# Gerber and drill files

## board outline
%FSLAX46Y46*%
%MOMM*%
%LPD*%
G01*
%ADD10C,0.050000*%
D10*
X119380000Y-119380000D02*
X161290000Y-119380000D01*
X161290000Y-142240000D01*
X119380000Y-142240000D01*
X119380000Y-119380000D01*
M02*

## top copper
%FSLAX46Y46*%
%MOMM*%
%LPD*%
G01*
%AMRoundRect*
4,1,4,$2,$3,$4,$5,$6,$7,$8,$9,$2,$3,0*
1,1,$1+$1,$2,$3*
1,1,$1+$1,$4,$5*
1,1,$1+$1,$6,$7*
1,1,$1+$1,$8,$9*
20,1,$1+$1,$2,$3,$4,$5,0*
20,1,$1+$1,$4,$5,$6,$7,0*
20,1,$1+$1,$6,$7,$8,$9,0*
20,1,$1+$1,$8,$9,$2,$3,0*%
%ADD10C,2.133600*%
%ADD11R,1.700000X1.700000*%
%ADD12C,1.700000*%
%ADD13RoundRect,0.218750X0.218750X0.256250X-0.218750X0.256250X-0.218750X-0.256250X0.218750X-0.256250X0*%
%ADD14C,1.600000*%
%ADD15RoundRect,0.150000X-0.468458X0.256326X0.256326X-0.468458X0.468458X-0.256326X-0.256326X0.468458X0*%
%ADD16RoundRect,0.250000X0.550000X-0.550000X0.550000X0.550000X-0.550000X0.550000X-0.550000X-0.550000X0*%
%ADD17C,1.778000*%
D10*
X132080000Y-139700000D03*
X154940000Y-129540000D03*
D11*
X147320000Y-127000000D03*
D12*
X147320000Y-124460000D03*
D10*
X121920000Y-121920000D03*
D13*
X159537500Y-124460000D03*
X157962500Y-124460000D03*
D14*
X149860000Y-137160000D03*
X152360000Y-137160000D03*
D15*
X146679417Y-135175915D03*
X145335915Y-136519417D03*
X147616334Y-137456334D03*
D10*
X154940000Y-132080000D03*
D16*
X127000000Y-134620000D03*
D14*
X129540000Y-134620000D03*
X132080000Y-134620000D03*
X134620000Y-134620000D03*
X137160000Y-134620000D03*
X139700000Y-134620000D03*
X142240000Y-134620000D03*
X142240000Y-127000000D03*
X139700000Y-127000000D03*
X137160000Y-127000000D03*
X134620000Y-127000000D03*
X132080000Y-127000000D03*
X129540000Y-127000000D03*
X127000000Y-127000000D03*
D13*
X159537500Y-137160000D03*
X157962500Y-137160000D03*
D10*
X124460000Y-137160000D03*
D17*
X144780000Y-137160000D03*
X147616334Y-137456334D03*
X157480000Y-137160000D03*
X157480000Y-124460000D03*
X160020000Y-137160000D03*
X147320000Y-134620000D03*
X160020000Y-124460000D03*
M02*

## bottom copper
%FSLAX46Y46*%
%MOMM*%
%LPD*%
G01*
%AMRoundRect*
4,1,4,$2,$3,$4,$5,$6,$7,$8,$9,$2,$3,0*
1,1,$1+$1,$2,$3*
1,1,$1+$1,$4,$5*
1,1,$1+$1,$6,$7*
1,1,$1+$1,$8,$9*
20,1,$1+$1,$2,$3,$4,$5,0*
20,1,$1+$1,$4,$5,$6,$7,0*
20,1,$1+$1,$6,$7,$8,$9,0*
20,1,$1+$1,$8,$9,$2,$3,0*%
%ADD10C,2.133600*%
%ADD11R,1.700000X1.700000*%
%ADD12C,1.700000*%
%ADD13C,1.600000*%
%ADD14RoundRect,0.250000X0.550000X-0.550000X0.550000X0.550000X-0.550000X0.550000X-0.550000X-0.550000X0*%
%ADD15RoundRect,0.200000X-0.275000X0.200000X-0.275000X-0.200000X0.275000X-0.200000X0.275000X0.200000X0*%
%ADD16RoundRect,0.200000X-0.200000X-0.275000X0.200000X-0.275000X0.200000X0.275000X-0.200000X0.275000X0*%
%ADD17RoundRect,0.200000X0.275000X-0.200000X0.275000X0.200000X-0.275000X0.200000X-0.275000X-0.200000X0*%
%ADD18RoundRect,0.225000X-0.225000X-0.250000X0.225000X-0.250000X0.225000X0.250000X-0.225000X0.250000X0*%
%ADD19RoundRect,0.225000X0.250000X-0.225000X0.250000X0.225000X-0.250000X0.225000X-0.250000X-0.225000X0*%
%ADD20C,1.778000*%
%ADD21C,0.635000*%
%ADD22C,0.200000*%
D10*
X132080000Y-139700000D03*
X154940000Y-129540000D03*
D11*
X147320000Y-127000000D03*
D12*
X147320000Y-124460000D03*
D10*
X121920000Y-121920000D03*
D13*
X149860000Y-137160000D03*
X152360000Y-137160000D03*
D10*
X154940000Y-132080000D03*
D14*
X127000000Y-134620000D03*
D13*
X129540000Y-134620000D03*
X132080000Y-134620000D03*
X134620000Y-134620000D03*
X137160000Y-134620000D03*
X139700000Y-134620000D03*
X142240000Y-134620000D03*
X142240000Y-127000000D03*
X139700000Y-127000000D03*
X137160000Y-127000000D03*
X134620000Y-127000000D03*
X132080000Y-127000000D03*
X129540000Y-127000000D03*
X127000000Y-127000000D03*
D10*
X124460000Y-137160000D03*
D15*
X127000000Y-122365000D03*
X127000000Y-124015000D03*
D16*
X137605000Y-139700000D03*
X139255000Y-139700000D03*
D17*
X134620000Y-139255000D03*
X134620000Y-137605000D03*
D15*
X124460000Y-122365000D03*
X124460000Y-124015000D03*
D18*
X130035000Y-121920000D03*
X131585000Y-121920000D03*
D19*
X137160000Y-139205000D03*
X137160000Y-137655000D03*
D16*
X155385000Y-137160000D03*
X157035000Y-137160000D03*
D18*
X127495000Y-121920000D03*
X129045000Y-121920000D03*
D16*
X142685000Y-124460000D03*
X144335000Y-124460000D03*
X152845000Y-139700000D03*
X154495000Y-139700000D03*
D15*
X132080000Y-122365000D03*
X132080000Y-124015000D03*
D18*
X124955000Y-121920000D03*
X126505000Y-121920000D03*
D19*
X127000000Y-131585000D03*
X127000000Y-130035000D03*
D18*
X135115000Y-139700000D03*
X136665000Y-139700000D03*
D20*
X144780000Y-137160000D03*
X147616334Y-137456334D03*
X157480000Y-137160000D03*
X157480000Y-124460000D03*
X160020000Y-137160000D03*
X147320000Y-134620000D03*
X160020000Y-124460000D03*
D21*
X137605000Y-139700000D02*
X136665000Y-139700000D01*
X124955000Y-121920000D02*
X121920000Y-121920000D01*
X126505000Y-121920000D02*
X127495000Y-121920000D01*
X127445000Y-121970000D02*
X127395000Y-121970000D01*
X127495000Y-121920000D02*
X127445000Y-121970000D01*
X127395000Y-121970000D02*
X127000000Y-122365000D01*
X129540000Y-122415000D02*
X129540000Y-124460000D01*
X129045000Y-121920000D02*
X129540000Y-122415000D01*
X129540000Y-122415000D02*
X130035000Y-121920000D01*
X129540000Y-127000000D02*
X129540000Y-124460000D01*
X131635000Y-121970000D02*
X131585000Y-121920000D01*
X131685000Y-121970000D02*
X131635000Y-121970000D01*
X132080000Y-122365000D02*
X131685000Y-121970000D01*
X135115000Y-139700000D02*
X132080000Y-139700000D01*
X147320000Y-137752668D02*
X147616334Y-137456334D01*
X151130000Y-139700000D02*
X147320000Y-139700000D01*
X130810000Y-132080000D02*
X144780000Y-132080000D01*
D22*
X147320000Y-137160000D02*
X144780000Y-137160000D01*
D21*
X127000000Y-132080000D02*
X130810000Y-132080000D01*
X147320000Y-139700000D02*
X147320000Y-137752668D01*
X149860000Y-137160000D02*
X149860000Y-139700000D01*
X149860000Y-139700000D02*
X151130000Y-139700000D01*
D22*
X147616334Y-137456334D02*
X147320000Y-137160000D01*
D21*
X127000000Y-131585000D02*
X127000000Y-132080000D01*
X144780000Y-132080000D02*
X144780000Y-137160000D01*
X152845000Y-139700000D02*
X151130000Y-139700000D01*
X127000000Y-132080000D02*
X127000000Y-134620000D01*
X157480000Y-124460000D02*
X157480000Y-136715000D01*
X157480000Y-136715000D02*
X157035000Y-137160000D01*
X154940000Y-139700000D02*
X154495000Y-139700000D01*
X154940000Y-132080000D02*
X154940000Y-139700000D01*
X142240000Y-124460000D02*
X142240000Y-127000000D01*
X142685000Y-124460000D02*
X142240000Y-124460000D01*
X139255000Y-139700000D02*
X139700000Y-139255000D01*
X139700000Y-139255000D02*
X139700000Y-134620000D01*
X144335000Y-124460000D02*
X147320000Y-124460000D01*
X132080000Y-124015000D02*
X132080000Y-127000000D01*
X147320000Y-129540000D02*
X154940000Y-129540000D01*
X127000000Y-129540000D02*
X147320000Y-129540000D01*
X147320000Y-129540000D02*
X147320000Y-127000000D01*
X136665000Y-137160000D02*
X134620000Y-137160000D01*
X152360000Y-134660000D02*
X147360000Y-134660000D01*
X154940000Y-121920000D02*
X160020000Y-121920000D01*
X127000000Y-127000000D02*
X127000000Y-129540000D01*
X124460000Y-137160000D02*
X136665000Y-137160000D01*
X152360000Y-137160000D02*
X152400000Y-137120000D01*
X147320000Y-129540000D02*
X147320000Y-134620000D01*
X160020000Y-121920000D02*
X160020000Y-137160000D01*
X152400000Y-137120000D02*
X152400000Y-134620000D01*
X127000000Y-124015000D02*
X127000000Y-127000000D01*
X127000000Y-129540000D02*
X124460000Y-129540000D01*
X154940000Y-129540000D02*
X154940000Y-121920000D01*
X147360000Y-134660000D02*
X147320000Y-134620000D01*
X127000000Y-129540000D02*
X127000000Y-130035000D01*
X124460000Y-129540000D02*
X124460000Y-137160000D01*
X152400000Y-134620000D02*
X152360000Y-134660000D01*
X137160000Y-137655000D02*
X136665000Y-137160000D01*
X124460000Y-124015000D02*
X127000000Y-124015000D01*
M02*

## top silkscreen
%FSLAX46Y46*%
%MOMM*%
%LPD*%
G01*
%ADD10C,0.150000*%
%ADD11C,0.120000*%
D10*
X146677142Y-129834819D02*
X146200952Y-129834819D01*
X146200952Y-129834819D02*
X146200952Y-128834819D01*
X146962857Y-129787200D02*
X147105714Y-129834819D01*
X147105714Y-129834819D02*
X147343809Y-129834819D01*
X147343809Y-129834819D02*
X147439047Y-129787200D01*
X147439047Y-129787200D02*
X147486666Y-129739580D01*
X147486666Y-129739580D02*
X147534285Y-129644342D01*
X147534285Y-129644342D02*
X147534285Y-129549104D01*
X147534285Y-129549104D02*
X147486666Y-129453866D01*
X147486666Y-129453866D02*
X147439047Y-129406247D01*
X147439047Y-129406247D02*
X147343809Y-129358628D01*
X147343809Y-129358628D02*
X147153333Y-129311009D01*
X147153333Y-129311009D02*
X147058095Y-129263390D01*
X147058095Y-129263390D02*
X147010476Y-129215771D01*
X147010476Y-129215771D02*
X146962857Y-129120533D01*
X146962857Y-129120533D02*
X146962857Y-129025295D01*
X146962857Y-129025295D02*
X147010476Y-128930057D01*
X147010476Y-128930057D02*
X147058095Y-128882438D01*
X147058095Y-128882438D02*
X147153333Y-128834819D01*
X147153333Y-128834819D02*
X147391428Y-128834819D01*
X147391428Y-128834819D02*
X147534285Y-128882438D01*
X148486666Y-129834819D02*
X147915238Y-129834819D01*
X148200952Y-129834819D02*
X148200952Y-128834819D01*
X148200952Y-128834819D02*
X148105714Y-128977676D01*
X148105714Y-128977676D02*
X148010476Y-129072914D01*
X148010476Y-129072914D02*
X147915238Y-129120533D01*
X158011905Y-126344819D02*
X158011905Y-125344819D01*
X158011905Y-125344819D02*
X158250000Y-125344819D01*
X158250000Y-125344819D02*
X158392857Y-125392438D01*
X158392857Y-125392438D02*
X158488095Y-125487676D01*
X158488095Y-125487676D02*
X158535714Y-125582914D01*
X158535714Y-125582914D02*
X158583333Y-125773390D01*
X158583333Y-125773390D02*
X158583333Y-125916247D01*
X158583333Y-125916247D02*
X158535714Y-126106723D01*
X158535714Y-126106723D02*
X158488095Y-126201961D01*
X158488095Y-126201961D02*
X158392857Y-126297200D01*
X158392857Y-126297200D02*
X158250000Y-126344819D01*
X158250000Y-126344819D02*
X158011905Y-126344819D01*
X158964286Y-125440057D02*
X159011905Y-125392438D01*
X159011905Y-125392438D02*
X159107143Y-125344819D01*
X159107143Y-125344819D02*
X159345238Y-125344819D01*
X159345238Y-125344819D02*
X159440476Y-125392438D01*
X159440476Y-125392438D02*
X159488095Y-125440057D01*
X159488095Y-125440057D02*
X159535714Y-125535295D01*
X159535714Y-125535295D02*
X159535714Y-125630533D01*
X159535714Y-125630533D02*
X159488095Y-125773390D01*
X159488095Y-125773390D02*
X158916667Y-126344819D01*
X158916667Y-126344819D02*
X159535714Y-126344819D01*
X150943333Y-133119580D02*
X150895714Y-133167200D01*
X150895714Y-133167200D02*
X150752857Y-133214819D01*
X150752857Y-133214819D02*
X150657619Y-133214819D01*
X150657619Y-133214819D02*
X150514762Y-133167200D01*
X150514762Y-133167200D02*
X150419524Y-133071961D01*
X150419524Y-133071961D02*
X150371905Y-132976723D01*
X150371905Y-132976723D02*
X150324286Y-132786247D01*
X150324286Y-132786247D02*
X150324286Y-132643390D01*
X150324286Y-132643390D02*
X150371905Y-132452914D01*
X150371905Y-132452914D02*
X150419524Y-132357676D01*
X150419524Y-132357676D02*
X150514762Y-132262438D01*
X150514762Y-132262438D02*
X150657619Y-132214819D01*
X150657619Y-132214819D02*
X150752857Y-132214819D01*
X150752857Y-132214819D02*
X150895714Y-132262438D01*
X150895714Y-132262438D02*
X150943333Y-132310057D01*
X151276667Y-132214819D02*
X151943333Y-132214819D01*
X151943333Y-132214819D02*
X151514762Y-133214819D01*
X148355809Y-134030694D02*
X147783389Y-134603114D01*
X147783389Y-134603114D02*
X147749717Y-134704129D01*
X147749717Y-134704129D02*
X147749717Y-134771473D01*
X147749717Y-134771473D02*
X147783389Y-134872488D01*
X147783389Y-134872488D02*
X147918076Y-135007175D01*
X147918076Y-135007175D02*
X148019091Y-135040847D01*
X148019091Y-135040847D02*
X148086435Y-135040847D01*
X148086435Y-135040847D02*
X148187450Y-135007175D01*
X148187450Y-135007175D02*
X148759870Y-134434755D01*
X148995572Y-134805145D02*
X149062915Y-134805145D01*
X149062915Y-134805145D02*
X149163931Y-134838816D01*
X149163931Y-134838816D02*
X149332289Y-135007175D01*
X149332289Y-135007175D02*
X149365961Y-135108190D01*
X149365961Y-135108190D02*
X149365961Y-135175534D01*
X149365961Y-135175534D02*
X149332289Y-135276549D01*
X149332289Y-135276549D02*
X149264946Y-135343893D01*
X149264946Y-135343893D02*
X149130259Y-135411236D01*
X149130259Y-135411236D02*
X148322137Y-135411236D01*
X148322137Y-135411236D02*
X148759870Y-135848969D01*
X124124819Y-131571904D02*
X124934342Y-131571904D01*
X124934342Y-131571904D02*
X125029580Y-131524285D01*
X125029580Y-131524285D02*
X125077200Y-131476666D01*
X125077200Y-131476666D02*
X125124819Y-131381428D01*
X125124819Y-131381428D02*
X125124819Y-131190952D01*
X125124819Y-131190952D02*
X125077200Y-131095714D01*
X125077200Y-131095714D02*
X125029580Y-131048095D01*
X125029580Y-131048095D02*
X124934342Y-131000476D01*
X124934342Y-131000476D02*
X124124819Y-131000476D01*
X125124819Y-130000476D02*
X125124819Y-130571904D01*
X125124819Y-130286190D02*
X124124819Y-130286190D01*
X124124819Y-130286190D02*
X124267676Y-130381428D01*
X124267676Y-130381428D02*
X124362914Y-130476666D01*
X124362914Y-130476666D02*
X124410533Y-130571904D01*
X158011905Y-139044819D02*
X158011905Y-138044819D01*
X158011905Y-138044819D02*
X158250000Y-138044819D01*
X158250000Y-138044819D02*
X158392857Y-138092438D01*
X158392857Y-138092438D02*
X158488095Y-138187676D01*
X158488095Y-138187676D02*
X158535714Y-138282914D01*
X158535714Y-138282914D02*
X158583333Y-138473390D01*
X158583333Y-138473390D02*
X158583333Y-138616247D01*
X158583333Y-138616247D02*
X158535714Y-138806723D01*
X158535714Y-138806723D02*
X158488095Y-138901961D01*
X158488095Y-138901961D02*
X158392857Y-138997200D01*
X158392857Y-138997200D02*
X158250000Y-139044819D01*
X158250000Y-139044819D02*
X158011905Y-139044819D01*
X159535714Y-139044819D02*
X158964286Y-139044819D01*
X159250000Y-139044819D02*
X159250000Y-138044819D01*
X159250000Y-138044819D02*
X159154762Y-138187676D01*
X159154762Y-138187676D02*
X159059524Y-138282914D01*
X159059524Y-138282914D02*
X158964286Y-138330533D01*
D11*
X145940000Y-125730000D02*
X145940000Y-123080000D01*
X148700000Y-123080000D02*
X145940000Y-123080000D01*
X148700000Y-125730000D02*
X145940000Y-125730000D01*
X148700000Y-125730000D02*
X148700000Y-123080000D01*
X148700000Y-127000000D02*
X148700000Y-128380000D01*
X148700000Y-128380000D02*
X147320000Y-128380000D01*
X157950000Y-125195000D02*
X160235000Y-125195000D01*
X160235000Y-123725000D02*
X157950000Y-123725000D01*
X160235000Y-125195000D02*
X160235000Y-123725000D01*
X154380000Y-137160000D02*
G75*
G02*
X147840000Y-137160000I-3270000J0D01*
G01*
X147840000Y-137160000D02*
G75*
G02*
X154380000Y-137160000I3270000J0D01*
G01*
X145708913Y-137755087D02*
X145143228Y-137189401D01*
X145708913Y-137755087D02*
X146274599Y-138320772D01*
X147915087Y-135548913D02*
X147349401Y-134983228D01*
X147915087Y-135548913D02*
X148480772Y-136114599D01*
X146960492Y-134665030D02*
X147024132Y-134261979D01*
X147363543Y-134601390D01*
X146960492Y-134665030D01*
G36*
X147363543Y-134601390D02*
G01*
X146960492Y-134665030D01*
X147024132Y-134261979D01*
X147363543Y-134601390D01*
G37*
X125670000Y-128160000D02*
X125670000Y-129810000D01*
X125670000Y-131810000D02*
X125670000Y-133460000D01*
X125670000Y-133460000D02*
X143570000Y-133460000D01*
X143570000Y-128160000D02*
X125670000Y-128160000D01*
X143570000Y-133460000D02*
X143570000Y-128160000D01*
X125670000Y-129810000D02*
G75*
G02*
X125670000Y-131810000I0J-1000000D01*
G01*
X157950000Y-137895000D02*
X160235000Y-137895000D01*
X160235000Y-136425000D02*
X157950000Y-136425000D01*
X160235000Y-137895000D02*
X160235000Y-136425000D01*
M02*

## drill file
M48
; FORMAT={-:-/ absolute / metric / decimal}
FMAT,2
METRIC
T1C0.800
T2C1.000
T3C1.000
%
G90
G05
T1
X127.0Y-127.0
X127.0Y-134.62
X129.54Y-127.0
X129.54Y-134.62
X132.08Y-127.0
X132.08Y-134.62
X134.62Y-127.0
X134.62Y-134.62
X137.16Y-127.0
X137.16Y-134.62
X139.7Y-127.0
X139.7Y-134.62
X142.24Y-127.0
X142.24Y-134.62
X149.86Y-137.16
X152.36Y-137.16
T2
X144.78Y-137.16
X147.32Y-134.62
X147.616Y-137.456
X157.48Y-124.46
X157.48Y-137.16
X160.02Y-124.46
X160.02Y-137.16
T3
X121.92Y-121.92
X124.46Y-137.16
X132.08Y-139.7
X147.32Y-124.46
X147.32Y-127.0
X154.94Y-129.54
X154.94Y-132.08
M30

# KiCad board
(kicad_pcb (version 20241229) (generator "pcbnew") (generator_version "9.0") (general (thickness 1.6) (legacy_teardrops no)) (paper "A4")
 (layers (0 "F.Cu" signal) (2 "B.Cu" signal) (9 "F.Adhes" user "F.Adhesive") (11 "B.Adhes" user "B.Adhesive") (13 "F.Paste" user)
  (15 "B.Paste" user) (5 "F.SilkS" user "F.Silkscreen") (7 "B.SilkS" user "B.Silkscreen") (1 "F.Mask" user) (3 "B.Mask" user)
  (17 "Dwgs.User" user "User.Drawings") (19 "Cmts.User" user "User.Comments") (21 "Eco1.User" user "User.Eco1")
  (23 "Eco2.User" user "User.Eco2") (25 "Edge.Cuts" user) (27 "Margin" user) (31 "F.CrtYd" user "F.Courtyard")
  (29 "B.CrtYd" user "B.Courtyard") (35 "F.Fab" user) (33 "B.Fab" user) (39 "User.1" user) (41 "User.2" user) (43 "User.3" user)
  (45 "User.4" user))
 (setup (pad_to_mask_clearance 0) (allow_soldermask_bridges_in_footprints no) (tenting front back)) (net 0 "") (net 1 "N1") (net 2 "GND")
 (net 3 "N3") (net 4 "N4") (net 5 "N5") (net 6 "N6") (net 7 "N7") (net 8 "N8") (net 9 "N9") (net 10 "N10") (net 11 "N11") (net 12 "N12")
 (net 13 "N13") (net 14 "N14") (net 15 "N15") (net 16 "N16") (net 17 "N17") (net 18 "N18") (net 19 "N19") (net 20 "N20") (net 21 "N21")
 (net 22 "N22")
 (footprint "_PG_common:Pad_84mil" (layer "F.Cu") (at 132.08 139.7)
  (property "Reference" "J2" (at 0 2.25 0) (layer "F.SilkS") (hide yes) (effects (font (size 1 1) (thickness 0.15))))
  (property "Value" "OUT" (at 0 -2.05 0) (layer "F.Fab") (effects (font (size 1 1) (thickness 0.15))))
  (pad "1" thru_hole circle (at 0 0) (size 2.1336 2.1336) (drill 1) (layers "*.Cu" "*.Mask") (remove_unused_layers no) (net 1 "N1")))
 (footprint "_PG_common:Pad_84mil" (layer "F.Cu") (at 154.94 129.54)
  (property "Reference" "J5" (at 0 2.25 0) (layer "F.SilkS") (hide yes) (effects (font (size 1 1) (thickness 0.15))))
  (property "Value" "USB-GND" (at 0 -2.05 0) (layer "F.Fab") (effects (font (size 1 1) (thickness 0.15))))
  (pad "1" thru_hole circle (at 0 0) (size 2.1336 2.1336) (drill 1) (layers "*.Cu" "*.Mask") (remove_unused_layers no) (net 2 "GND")))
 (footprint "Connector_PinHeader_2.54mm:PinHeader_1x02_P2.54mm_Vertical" (layer "F.Cu") (at 147.32 127 180)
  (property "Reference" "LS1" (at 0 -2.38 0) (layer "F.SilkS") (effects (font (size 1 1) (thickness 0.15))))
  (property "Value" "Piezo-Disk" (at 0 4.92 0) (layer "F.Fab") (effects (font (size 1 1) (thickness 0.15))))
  (fp_line (start 1.38 1.27) (end 1.38 3.92) (stroke (width 0.12) (type solid)) (layer "F.SilkS"))
  (fp_line (start -1.38 3.92) (end 1.38 3.92) (stroke (width 0.12) (type solid)) (layer "F.SilkS"))
  (fp_line (start -1.38 1.27) (end 1.38 1.27) (stroke (width 0.12) (type solid)) (layer "F.SilkS"))
  (fp_line (start -1.38 1.27) (end -1.38 3.92) (stroke (width 0.12) (type solid)) (layer "F.SilkS"))
  (fp_line (start -1.38 0) (end -1.38 -1.38) (stroke (width 0.12) (type solid)) (layer "F.SilkS"))
  (fp_line (start -1.38 -1.38) (end 0 -1.38) (stroke (width 0.12) (type solid)) (layer "F.SilkS"))
  (pad "1" thru_hole rect (at 0 0 180) (size 1.7 1.7) (drill 1) (layers "*.Cu" "*.Mask") (remove_unused_layers no) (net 2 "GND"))
  (pad "2" thru_hole circle (at 0 2.54 180) (size 1.7 1.7) (drill 1) (layers "*.Cu" "*.Mask") (remove_unused_layers no) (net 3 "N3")))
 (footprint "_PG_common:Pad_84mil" (layer "F.Cu") (at 121.92 121.92)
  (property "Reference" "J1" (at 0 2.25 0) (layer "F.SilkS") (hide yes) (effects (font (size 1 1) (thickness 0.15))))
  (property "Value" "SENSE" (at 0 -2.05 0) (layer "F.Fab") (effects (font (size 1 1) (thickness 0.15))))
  (pad "1" thru_hole circle (at 0 0) (size 2.1336 2.1336) (drill 1) (layers "*.Cu" "*.Mask") (remove_unused_layers no) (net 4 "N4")))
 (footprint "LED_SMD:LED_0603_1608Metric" (layer "F.Cu") (at 158.75 124.46 180)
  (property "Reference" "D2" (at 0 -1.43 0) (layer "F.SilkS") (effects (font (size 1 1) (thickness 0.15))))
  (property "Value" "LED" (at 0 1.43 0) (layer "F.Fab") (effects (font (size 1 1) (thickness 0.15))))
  (fp_line (start 0.8 -0.735) (end -1.485 -0.735) (stroke (width 0.12) (type solid)) (layer "F.SilkS"))
  (fp_line (start -1.485 0.735) (end 0.8 0.735) (stroke (width 0.12) (type solid)) (layer "F.SilkS"))
  (fp_line (start -1.485 -0.735) (end -1.485 0.735) (stroke (width 0.12) (type solid)) (layer "F.SilkS"))
  (pad "1" smd roundrect (at -0.7875 0 180) (size 0.875 0.95) (layers "F.Cu" "F.Mask" "F.Paste") (roundrect_rratio 0.25) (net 2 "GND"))
  (pad "2" smd roundrect (at 0.7875 0 180) (size 0.875 0.95) (layers "F.Cu" "F.Mask" "F.Paste") (roundrect_rratio 0.25) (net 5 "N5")))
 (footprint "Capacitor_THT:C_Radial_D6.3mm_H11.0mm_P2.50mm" (layer "F.Cu") (at 149.86 137.16)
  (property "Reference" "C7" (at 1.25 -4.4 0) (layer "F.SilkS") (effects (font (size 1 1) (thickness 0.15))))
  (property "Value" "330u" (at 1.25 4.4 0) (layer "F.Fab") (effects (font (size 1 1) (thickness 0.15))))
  (fp_circle (center 1.25 0) (end 4.52 0) (stroke (width 0.12) (type solid)) (fill no) (layer "F.SilkS"))
  (pad "1" thru_hole circle (at 0 0) (size 1.6 1.6) (drill 0.8) (layers "*.Cu" "*.Mask") (remove_unused_layers no) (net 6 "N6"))
  (pad "2" thru_hole circle (at 2.5 0) (size 1.6 1.6) (drill 0.8) (layers "*.Cu" "*.Mask") (remove_unused_layers no) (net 2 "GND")))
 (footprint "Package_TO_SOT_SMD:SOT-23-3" (layer "F.Cu") (at 146.812 136.652 -45)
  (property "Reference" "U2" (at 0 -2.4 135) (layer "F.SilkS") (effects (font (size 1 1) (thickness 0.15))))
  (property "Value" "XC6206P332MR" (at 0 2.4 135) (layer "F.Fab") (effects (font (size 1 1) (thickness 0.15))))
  (fp_line (start 0 1.560001) (end -0.8 1.56) (stroke (width 0.12) (type solid)) (layer "F.SilkS"))
  (fp_line (start 0 1.560001) (end 0.8 1.56) (stroke (width 0.12) (type solid)) (layer "F.SilkS"))
  (fp_line (start 0 -1.560001) (end -0.8 -1.56) (stroke (width 0.12) (type solid)) (layer "F.SilkS"))
  (fp_line (start 0 -1.560001) (end 0.8 -1.56) (stroke (width 0.12) (type solid)) (layer "F.SilkS"))
  (fp_poly (pts (xy -1.3 -1.51) (xy -1.54 -1.84) (xy -1.06 -1.84)) (stroke (width 0.12) (type solid)) (fill yes) (layer "F.SilkS"))
  (pad "1" smd roundrect (at -1.1375 -0.949999 315) (size 1.325 0.6) (layers "F.Cu" "F.Mask" "F.Paste") (roundrect_rratio 0.25)
   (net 2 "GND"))
  (pad "2" smd roundrect (at -1.1375 0.949999 315) (size 1.325 0.6) (layers "F.Cu" "F.Mask" "F.Paste") (roundrect_rratio 0.25) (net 6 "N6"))
  (pad "3" smd roundrect (at 1.1375 0 315) (size 1.325 0.6) (layers "F.Cu" "F.Mask" "F.Paste") (roundrect_rratio 0.25) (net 6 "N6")))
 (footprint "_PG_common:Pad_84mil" (layer "F.Cu") (at 154.94 132.08)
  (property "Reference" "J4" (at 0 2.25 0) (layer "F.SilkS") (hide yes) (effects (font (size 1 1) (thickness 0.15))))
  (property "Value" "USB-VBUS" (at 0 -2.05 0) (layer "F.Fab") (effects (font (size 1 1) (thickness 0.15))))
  (pad "1" thru_hole circle (at 0 0) (size 2.1336 2.1336) (drill 1) (layers "*.Cu" "*.Mask") (remove_unused_layers no) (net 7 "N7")))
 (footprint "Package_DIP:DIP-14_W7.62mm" (layer "F.Cu") (at 127 134.62 90)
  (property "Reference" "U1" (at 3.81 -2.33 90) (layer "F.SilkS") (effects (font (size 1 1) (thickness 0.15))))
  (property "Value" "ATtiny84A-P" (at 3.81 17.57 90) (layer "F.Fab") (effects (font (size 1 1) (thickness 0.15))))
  (fp_line (start 6.46 -1.33) (end 4.81 -1.33) (stroke (width 0.12) (type solid)) (layer "F.SilkS"))
  (fp_line (start 2.81 -1.33) (end 1.16 -1.33) (stroke (width 0.12) (type solid)) (layer "F.SilkS"))
  (fp_line (start 1.16 -1.33) (end 1.16 16.57) (stroke (width 0.12) (type solid)) (layer "F.SilkS"))
  (fp_line (start 6.46 16.57) (end 6.46 -1.33) (stroke (width 0.12) (type solid)) (layer "F.SilkS"))
  (fp_line (start 1.16 16.57) (end 6.46 16.57) (stroke (width 0.12) (type solid)) (layer "F.SilkS"))
  (fp_arc (start 4.81 -1.33) (mid 3.81 -0.33) (end 2.81 -1.33) (stroke (width 0.12) (type solid)) (layer "F.SilkS"))
  (pad "1" thru_hole roundrect (at 0 0 90) (size 1.6 1.6) (drill 0.8) (layers "*.Cu" "*.Mask") (remove_unused_layers no)
   (roundrect_rratio 0.15625) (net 6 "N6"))
  (pad "2" thru_hole circle (at 0 2.54 90) (size 1.6 1.6) (drill 0.8) (layers "*.Cu" "*.Mask") (remove_unused_layers no) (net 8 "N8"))
  (pad "3" thru_hole circle (at 0 5.08 90) (size 1.6 1.6) (drill 0.8) (layers "*.Cu" "*.Mask") (remove_unused_layers no) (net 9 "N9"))
  (pad "4" thru_hole circle (at 0 7.62 90) (size 1.6 1.6) (drill 0.8) (layers "*.Cu" "*.Mask") (remove_unused_layers no) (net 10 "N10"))
  (pad "5" thru_hole circle (at 0 10.16 90) (size 1.6 1.6) (drill 0.8) (layers "*.Cu" "*.Mask") (remove_unused_layers no) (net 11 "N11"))
  (pad "6" thru_hole circle (at 0 12.7 90) (size 1.6 1.6) (drill 0.8) (layers "*.Cu" "*.Mask") (remove_unused_layers no) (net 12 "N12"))
  (pad "7" thru_hole circle (at 0 15.24 90) (size 1.6 1.6) (drill 0.8) (layers "*.Cu" "*.Mask") (remove_unused_layers no) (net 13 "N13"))
  (pad "8" thru_hole circle (at 7.62 15.24 90) (size 1.6 1.6) (drill 0.8) (layers "*.Cu" "*.Mask") (remove_unused_layers no) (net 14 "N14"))
  (pad "9" thru_hole circle (at 7.62 12.7 90) (size 1.6 1.6) (drill 0.8) (layers "*.Cu" "*.Mask") (remove_unused_layers no) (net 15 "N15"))
  (pad "10" thru_hole circle (at 7.62 10.16 90) (size 1.6 1.6) (drill 0.8) (layers "*.Cu" "*.Mask") (remove_unused_layers no) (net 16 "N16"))
  (pad "11" thru_hole circle (at 7.62 7.62 90) (size 1.6 1.6) (drill 0.8) (layers "*.Cu" "*.Mask") (remove_unused_layers no) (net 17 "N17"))
  (pad "12" thru_hole circle (at 7.62 5.08 90) (size 1.6 1.6) (drill 0.8) (layers "*.Cu" "*.Mask") (remove_unused_layers no) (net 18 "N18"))
  (pad "13" thru_hole circle (at 7.62 2.54 90) (size 1.6 1.6) (drill 0.8) (layers "*.Cu" "*.Mask") (remove_unused_layers no) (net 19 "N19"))
  (pad "14" thru_hole circle (at 7.62 0 90) (size 1.6 1.6) (drill 0.8) (layers "*.Cu" "*.Mask") (remove_unused_layers no) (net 2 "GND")))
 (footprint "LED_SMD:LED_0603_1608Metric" (layer "F.Cu") (at 158.75 137.16 180)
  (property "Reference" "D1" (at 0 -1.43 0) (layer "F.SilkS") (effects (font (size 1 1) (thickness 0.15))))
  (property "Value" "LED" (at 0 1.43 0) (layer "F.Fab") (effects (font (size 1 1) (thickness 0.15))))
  (fp_line (start 0.8 -0.735) (end -1.485 -0.735) (stroke (width 0.12) (type solid)) (layer "F.SilkS"))
  (fp_line (start -1.485 0.735) (end 0.8 0.735) (stroke (width 0.12) (type solid)) (layer "F.SilkS"))
  (fp_line (start -1.485 -0.735) (end -1.485 0.735) (stroke (width 0.12) (type solid)) (layer "F.SilkS"))
  (pad "1" smd roundrect (at -0.7875 0 180) (size 0.875 0.95) (layers "F.Cu" "F.Mask" "F.Paste") (roundrect_rratio 0.25) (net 2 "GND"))
  (pad "2" smd roundrect (at 0.7875 0 180) (size 0.875 0.95) (layers "F.Cu" "F.Mask" "F.Paste") (roundrect_rratio 0.25) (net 5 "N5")))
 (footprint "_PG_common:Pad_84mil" (layer "F.Cu") (at 124.46 137.16)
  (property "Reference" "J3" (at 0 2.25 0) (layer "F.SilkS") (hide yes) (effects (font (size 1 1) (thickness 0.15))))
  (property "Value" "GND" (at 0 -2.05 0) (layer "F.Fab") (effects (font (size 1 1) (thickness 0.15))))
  (pad "1" thru_hole circle (at 0 0) (size 2.1336 2.1336) (drill 1) (layers "*.Cu" "*.Mask") (remove_unused_layers no) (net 2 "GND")))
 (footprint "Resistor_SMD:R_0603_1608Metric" (layer "B.Cu") (at 127 123.19 -90)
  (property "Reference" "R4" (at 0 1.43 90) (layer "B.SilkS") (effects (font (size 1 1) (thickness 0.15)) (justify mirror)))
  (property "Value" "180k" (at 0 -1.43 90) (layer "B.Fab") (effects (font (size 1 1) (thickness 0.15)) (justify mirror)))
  (pad "1" smd roundrect (at -0.825 0 270) (size 0.8 0.95) (layers "B.Cu" "B.Mask" "B.Paste") (roundrect_rratio 0.25) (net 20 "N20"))
  (pad "2" smd roundrect (at 0.825 0 270) (size 0.8 0.95) (layers "B.Cu" "B.Mask" "B.Paste") (roundrect_rratio 0.25) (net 2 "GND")))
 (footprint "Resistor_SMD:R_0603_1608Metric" (layer "B.Cu") (at 138.43 139.7)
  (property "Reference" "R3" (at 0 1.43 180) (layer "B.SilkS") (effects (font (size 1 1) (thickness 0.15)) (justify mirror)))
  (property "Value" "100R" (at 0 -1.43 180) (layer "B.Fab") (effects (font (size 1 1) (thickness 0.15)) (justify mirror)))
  (pad "1" smd roundrect (at -0.825 0) (size 0.8 0.95) (layers "B.Cu" "B.Mask" "B.Paste") (roundrect_rratio 0.25) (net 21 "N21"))
  (pad "2" smd roundrect (at 0.825 0) (size 0.8 0.95) (layers "B.Cu" "B.Mask" "B.Paste") (roundrect_rratio 0.25) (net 12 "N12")))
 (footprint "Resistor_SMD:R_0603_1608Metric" (layer "B.Cu") (at 134.62 138.43 90)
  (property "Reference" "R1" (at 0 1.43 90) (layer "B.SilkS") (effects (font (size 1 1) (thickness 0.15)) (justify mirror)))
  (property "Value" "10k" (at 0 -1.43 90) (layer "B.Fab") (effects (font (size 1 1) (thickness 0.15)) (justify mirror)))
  (pad "1" smd roundrect (at -0.825 0 90) (size 0.8 0.95) (layers "B.Cu" "B.Mask" "B.Paste") (roundrect_rratio 0.25) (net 1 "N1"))
  (pad "2" smd roundrect (at 0.825 0 90) (size 0.8 0.95) (layers "B.Cu" "B.Mask" "B.Paste") (roundrect_rratio 0.25) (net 2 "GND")))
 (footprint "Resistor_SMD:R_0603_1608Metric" (layer "B.Cu") (at 124.46 123.19 -90)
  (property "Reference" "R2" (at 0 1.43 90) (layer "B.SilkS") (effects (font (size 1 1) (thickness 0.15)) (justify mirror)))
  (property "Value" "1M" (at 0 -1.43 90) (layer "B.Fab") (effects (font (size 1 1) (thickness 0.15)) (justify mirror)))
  (pad "1" smd roundrect (at -0.825 0 270) (size 0.8 0.95) (layers "B.Cu" "B.Mask" "B.Paste") (roundrect_rratio 0.25) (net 4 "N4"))
  (pad "2" smd roundrect (at 0.825 0 270) (size 0.8 0.95) (layers "B.Cu" "B.Mask" "B.Paste") (roundrect_rratio 0.25) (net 2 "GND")))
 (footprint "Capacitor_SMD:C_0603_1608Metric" (layer "B.Cu") (at 130.81 121.92)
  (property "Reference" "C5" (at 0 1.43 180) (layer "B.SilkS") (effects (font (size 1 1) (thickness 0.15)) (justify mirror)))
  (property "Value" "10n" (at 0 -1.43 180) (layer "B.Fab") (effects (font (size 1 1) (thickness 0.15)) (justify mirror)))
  (pad "1" smd roundrect (at -0.775 0) (size 0.9 0.95) (layers "B.Cu" "B.Mask" "B.Paste") (roundrect_rratio 0.25) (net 19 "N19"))
  (pad "2" smd roundrect (at 0.775 0) (size 0.9 0.95) (layers "B.Cu" "B.Mask" "B.Paste") (roundrect_rratio 0.25) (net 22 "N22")))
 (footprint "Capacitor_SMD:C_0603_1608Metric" (layer "B.Cu") (at 137.16 138.43 90)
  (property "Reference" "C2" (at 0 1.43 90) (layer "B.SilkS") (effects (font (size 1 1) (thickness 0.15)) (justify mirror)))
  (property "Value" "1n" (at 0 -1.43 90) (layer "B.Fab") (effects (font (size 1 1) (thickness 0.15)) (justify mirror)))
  (pad "1" smd roundrect (at -0.775 0 90) (size 0.9 0.95) (layers "B.Cu" "B.Mask" "B.Paste") (roundrect_rratio 0.25) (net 21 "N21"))
  (pad "2" smd roundrect (at 0.775 0 90) (size 0.9 0.95) (layers "B.Cu" "B.Mask" "B.Paste") (roundrect_rratio 0.25) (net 2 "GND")))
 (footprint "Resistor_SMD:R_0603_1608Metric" (layer "B.Cu") (at 156.21 137.16)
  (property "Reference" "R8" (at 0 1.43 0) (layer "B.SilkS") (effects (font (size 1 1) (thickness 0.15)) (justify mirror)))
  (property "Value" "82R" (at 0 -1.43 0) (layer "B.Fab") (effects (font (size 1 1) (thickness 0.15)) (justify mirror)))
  (pad "1" smd roundrect (at -0.825 0) (size 0.8 0.95) (layers "B.Cu" "B.Mask" "B.Paste") (roundrect_rratio 0.25) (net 7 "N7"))
  (pad "2" smd roundrect (at 0.825 0) (size 0.8 0.95) (layers "B.Cu" "B.Mask" "B.Paste") (roundrect_rratio 0.25) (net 5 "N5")))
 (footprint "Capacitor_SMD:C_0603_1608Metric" (layer "B.Cu") (at 128.27 121.92)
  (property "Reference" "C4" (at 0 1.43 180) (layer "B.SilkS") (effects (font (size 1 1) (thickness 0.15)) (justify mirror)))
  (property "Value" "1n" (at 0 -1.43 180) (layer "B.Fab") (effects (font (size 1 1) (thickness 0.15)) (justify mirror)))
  (pad "1" smd roundrect (at -0.775 0) (size 0.9 0.95) (layers "B.Cu" "B.Mask" "B.Paste") (roundrect_rratio 0.25) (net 20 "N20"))
  (pad "2" smd roundrect (at 0.775 0) (size 0.9 0.95) (layers "B.Cu" "B.Mask" "B.Paste") (roundrect_rratio 0.25) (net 19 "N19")))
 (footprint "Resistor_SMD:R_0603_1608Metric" (layer "B.Cu") (at 143.51 124.46)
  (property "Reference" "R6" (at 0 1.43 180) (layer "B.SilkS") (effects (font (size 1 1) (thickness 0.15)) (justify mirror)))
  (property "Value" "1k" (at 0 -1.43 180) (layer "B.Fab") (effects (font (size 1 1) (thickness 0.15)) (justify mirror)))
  (pad "1" smd roundrect (at -0.825 0) (size 0.8 0.95) (layers "B.Cu" "B.Mask" "B.Paste") (roundrect_rratio 0.25) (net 14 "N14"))
  (pad "2" smd roundrect (at 0.825 0) (size 0.8 0.95) (layers "B.Cu" "B.Mask" "B.Paste") (roundrect_rratio 0.25) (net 3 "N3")))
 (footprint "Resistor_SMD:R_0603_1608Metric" (layer "B.Cu") (at 153.67 139.7)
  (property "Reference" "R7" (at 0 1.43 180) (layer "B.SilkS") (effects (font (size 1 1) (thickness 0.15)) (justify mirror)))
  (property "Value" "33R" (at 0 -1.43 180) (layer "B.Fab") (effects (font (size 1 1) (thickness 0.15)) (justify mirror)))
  (pad "1" smd roundrect (at -0.825 0) (size 0.8 0.95) (layers "B.Cu" "B.Mask" "B.Paste") (roundrect_rratio 0.25) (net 6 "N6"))
  (pad "2" smd roundrect (at 0.825 0) (size 0.8 0.95) (layers "B.Cu" "B.Mask" "B.Paste") (roundrect_rratio 0.25) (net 7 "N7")))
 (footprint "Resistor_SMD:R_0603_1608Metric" (layer "B.Cu") (at 132.08 123.19 -90)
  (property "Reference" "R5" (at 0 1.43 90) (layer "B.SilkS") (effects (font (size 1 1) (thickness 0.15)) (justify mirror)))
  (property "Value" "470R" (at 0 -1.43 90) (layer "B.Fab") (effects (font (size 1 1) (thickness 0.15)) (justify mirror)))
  (pad "1" smd roundrect (at -0.825 0 270) (size 0.8 0.95) (layers "B.Cu" "B.Mask" "B.Paste") (roundrect_rratio 0.25) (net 22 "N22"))
  (pad "2" smd roundrect (at 0.825 0 270) (size 0.8 0.95) (layers "B.Cu" "B.Mask" "B.Paste") (roundrect_rratio 0.25) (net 18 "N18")))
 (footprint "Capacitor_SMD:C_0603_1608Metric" (layer "B.Cu") (at 125.73 121.92)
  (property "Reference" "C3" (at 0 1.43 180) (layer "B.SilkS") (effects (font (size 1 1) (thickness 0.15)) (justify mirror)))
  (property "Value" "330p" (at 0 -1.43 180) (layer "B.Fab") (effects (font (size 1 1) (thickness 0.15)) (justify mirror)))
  (pad "1" smd roundrect (at -0.775 0) (size 0.9 0.95) (layers "B.Cu" "B.Mask" "B.Paste") (roundrect_rratio 0.25) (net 4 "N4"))
  (pad "2" smd roundrect (at 0.775 0) (size 0.9 0.95) (layers "B.Cu" "B.Mask" "B.Paste") (roundrect_rratio 0.25) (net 20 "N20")))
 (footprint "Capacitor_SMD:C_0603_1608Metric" (layer "B.Cu") (at 127 130.81 90)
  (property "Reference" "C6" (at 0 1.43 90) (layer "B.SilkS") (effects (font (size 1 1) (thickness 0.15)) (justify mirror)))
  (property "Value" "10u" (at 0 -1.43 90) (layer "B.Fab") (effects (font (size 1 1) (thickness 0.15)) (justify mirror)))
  (pad "1" smd roundrect (at -0.775 0 90) (size 0.9 0.95) (layers "B.Cu" "B.Mask" "B.Paste") (roundrect_rratio 0.25) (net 6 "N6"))
  (pad "2" smd roundrect (at 0.775 0 90) (size 0.9 0.95) (layers "B.Cu" "B.Mask" "B.Paste") (roundrect_rratio 0.25) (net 2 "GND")))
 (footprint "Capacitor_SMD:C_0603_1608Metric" (layer "B.Cu") (at 135.89 139.7)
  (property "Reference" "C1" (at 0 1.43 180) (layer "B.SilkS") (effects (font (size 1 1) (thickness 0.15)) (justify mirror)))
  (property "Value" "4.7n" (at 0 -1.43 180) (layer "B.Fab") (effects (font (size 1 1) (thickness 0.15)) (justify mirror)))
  (pad "1" smd roundrect (at -0.775 0) (size 0.9 0.95) (layers "B.Cu" "B.Mask" "B.Paste") (roundrect_rratio 0.25) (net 1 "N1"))
  (pad "2" smd roundrect (at 0.775 0) (size 0.9 0.95) (layers "B.Cu" "B.Mask" "B.Paste") (roundrect_rratio 0.25) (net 21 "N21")))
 (gr_rect (start 119.38 119.38) (end 161.29 142.24) (stroke (width 0.05) (type default)) (fill no) (layer "Edge.Cuts"))
 (segment (start 137.605 139.7) (end 136.665 139.7) (width 0.635) (layer "B.Cu") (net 21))
 (segment (start 124.955 121.92) (end 121.92 121.92) (width 0.635) (layer "B.Cu") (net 4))
 (segment (start 126.505 121.92) (end 127.495 121.92) (width 0.635) (layer "B.Cu") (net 20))
 (segment (start 127.445 121.97) (end 127.395 121.97) (width 0.635) (layer "B.Cu") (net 20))
 (segment (start 127.495 121.92) (end 127.445 121.97) (width 0.635) (layer "B.Cu") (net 20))
 (segment (start 127.395 121.97) (end 127 122.365) (width 0.635) (layer "B.Cu") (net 20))
 (segment (start 129.54 122.415) (end 129.54 124.46) (width 0.635) (layer "B.Cu") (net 19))
 (segment (start 129.045 121.92) (end 129.54 122.415) (width 0.635) (layer "B.Cu") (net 19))
 (segment (start 129.54 122.415) (end 130.035 121.92) (width 0.635) (layer "B.Cu") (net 19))
 (segment (start 129.54 127) (end 129.54 124.46) (width 0.635) (layer "B.Cu") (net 19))
 (segment (start 131.635 121.97) (end 131.585 121.92) (width 0.635) (layer "B.Cu") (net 22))
 (segment (start 131.685 121.97) (end 131.635 121.97) (width 0.635) (layer "B.Cu") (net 22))
 (segment (start 132.08 122.365) (end 131.685 121.97) (width 0.635) (layer "B.Cu") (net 22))
 (segment (start 135.115 139.7) (end 132.08 139.7) (width 0.635) (layer "B.Cu") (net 1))
 (via (at 144.78 137.16) (size 1.778) (drill 1) (layers "F.Cu" "B.Cu") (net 6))
 (via (at 147.616334 137.456334) (size 1.778) (drill 1) (layers "F.Cu" "B.Cu") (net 6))
 (segment (start 147.32 137.752668) (end 147.616334 137.456334) (width 0.635) (layer "B.Cu") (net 6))
 (segment (start 151.13 139.7) (end 147.32 139.7) (width 0.635) (layer "B.Cu") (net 6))
 (segment (start 130.81 132.08) (end 144.78 132.08) (width 0.635) (layer "B.Cu") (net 6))
 (segment (start 147.32 137.16) (end 144.78 137.16) (width 0.2) (layer "B.Cu") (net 6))
 (segment (start 127 132.08) (end 130.81 132.08) (width 0.635) (layer "B.Cu") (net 6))
 (segment (start 147.32 139.7) (end 147.32 137.752668) (width 0.635) (layer "B.Cu") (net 6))
 (segment (start 149.86 137.16) (end 149.86 139.7) (width 0.635) (layer "B.Cu") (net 6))
 (segment (start 149.86 139.7) (end 151.13 139.7) (width 0.635) (layer "B.Cu") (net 6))
 (segment (start 147.616334 137.456334) (end 147.32 137.16) (width 0.2) (layer "B.Cu") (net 6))
 (segment (start 127 131.585) (end 127 132.08) (width 0.635) (layer "B.Cu") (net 6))
 (segment (start 144.78 132.08) (end 144.78 137.16) (width 0.635) (layer "B.Cu") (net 6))
 (segment (start 152.845 139.7) (end 151.13 139.7) (width 0.635) (layer "B.Cu") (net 6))
 (segment (start 127 132.08) (end 127 134.62) (width 0.635) (layer "B.Cu") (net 6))
 (via (at 157.48 137.16) (size 1.778) (drill 1) (layers "F.Cu" "B.Cu") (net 5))
 (via (at 157.48 124.46) (size 1.778) (drill 1) (layers "F.Cu" "B.Cu") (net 5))
 (segment (start 157.48 124.46) (end 157.48 136.715) (width 0.635) (layer "B.Cu") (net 5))
 (segment (start 157.48 136.715) (end 157.035 137.16) (width 0.635) (layer "B.Cu") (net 5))
 (segment (start 154.94 139.7) (end 154.495 139.7) (width 0.635) (layer "B.Cu") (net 7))
 (segment (start 154.94 132.08) (end 154.94 139.7) (width 0.635) (layer "B.Cu") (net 7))
 (segment (start 142.24 124.46) (end 142.24 127) (width 0.635) (layer "B.Cu") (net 14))
 (segment (start 142.685 124.46) (end 142.24 124.46) (width 0.635) (layer "B.Cu") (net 14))
 (segment (start 139.255 139.7) (end 139.7 139.255) (width 0.635) (layer "B.Cu") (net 12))
 (segment (start 139.7 139.255) (end 139.7 134.62) (width 0.635) (layer "B.Cu") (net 12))
 (segment (start 144.335 124.46) (end 147.32 124.46) (width 0.635) (layer "B.Cu") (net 3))
 (segment (start 132.08 124.015) (end 132.08 127) (width 0.635) (layer "B.Cu") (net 18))
 (via (at 160.02 137.16) (size 1.778) (drill 1) (layers "F.Cu" "B.Cu") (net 2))
 (via (at 147.32 134.62) (size 1.778) (drill 1) (layers "F.Cu" "B.Cu") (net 2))
 (via (at 160.02 124.46) (size 1.778) (drill 1) (layers "F.Cu" "B.Cu") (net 2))
 (segment (start 147.32 129.54) (end 154.94 129.54) (width 0.635) (layer "B.Cu") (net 2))
 (segment (start 127 129.54) (end 147.32 129.54) (width 0.635) (layer "B.Cu") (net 2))
 (segment (start 147.32 129.54) (end 147.32 127) (width 0.635) (layer "B.Cu") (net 2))
 (segment (start 136.665 137.16) (end 134.62 137.16) (width 0.635) (layer "B.Cu") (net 2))
 (segment (start 152.36 134.66) (end 147.36 134.66) (width 0.635) (layer "B.Cu") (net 2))
 (segment (start 154.94 121.92) (end 160.02 121.92) (width 0.635) (layer "B.Cu") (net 2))
 (segment (start 127 127) (end 127 129.54) (width 0.635) (layer "B.Cu") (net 2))
 (segment (start 124.46 137.16) (end 136.665 137.16) (width 0.635) (layer "B.Cu") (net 2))
 (segment (start 152.36 137.16) (end 152.4 137.12) (width 0.635) (layer "B.Cu") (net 2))
 (segment (start 147.32 129.54) (end 147.32 134.62) (width 0.635) (layer "B.Cu") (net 2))
 (segment (start 160.02 121.92) (end 160.02 137.16) (width 0.635) (layer "B.Cu") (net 2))
 (segment (start 152.4 137.12) (end 152.4 134.62) (width 0.635) (layer "B.Cu") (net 2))
 (segment (start 127 124.015) (end 127 127) (width 0.635) (layer "B.Cu") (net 2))
 (segment (start 127 129.54) (end 124.46 129.54) (width 0.635) (layer "B.Cu") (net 2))
 (segment (start 154.94 129.54) (end 154.94 121.92) (width 0.635) (layer "B.Cu") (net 2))
 (segment (start 147.36 134.66) (end 147.32 134.62) (width 0.635) (layer "B.Cu") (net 2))
 (segment (start 127 129.54) (end 127 130.035) (width 0.635) (layer "B.Cu") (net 2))
 (segment (start 124.46 129.54) (end 124.46 137.16) (width 0.635) (layer "B.Cu") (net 2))
 (segment (start 152.4 134.62) (end 152.36 134.66) (width 0.635) (layer "B.Cu") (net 2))
 (segment (start 137.16 137.655) (end 136.665 137.16) (width 0.635) (layer "B.Cu") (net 2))
 (segment (start 124.46 124.015) (end 127 124.015) (width 0.635) (layer "B.Cu") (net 2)))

